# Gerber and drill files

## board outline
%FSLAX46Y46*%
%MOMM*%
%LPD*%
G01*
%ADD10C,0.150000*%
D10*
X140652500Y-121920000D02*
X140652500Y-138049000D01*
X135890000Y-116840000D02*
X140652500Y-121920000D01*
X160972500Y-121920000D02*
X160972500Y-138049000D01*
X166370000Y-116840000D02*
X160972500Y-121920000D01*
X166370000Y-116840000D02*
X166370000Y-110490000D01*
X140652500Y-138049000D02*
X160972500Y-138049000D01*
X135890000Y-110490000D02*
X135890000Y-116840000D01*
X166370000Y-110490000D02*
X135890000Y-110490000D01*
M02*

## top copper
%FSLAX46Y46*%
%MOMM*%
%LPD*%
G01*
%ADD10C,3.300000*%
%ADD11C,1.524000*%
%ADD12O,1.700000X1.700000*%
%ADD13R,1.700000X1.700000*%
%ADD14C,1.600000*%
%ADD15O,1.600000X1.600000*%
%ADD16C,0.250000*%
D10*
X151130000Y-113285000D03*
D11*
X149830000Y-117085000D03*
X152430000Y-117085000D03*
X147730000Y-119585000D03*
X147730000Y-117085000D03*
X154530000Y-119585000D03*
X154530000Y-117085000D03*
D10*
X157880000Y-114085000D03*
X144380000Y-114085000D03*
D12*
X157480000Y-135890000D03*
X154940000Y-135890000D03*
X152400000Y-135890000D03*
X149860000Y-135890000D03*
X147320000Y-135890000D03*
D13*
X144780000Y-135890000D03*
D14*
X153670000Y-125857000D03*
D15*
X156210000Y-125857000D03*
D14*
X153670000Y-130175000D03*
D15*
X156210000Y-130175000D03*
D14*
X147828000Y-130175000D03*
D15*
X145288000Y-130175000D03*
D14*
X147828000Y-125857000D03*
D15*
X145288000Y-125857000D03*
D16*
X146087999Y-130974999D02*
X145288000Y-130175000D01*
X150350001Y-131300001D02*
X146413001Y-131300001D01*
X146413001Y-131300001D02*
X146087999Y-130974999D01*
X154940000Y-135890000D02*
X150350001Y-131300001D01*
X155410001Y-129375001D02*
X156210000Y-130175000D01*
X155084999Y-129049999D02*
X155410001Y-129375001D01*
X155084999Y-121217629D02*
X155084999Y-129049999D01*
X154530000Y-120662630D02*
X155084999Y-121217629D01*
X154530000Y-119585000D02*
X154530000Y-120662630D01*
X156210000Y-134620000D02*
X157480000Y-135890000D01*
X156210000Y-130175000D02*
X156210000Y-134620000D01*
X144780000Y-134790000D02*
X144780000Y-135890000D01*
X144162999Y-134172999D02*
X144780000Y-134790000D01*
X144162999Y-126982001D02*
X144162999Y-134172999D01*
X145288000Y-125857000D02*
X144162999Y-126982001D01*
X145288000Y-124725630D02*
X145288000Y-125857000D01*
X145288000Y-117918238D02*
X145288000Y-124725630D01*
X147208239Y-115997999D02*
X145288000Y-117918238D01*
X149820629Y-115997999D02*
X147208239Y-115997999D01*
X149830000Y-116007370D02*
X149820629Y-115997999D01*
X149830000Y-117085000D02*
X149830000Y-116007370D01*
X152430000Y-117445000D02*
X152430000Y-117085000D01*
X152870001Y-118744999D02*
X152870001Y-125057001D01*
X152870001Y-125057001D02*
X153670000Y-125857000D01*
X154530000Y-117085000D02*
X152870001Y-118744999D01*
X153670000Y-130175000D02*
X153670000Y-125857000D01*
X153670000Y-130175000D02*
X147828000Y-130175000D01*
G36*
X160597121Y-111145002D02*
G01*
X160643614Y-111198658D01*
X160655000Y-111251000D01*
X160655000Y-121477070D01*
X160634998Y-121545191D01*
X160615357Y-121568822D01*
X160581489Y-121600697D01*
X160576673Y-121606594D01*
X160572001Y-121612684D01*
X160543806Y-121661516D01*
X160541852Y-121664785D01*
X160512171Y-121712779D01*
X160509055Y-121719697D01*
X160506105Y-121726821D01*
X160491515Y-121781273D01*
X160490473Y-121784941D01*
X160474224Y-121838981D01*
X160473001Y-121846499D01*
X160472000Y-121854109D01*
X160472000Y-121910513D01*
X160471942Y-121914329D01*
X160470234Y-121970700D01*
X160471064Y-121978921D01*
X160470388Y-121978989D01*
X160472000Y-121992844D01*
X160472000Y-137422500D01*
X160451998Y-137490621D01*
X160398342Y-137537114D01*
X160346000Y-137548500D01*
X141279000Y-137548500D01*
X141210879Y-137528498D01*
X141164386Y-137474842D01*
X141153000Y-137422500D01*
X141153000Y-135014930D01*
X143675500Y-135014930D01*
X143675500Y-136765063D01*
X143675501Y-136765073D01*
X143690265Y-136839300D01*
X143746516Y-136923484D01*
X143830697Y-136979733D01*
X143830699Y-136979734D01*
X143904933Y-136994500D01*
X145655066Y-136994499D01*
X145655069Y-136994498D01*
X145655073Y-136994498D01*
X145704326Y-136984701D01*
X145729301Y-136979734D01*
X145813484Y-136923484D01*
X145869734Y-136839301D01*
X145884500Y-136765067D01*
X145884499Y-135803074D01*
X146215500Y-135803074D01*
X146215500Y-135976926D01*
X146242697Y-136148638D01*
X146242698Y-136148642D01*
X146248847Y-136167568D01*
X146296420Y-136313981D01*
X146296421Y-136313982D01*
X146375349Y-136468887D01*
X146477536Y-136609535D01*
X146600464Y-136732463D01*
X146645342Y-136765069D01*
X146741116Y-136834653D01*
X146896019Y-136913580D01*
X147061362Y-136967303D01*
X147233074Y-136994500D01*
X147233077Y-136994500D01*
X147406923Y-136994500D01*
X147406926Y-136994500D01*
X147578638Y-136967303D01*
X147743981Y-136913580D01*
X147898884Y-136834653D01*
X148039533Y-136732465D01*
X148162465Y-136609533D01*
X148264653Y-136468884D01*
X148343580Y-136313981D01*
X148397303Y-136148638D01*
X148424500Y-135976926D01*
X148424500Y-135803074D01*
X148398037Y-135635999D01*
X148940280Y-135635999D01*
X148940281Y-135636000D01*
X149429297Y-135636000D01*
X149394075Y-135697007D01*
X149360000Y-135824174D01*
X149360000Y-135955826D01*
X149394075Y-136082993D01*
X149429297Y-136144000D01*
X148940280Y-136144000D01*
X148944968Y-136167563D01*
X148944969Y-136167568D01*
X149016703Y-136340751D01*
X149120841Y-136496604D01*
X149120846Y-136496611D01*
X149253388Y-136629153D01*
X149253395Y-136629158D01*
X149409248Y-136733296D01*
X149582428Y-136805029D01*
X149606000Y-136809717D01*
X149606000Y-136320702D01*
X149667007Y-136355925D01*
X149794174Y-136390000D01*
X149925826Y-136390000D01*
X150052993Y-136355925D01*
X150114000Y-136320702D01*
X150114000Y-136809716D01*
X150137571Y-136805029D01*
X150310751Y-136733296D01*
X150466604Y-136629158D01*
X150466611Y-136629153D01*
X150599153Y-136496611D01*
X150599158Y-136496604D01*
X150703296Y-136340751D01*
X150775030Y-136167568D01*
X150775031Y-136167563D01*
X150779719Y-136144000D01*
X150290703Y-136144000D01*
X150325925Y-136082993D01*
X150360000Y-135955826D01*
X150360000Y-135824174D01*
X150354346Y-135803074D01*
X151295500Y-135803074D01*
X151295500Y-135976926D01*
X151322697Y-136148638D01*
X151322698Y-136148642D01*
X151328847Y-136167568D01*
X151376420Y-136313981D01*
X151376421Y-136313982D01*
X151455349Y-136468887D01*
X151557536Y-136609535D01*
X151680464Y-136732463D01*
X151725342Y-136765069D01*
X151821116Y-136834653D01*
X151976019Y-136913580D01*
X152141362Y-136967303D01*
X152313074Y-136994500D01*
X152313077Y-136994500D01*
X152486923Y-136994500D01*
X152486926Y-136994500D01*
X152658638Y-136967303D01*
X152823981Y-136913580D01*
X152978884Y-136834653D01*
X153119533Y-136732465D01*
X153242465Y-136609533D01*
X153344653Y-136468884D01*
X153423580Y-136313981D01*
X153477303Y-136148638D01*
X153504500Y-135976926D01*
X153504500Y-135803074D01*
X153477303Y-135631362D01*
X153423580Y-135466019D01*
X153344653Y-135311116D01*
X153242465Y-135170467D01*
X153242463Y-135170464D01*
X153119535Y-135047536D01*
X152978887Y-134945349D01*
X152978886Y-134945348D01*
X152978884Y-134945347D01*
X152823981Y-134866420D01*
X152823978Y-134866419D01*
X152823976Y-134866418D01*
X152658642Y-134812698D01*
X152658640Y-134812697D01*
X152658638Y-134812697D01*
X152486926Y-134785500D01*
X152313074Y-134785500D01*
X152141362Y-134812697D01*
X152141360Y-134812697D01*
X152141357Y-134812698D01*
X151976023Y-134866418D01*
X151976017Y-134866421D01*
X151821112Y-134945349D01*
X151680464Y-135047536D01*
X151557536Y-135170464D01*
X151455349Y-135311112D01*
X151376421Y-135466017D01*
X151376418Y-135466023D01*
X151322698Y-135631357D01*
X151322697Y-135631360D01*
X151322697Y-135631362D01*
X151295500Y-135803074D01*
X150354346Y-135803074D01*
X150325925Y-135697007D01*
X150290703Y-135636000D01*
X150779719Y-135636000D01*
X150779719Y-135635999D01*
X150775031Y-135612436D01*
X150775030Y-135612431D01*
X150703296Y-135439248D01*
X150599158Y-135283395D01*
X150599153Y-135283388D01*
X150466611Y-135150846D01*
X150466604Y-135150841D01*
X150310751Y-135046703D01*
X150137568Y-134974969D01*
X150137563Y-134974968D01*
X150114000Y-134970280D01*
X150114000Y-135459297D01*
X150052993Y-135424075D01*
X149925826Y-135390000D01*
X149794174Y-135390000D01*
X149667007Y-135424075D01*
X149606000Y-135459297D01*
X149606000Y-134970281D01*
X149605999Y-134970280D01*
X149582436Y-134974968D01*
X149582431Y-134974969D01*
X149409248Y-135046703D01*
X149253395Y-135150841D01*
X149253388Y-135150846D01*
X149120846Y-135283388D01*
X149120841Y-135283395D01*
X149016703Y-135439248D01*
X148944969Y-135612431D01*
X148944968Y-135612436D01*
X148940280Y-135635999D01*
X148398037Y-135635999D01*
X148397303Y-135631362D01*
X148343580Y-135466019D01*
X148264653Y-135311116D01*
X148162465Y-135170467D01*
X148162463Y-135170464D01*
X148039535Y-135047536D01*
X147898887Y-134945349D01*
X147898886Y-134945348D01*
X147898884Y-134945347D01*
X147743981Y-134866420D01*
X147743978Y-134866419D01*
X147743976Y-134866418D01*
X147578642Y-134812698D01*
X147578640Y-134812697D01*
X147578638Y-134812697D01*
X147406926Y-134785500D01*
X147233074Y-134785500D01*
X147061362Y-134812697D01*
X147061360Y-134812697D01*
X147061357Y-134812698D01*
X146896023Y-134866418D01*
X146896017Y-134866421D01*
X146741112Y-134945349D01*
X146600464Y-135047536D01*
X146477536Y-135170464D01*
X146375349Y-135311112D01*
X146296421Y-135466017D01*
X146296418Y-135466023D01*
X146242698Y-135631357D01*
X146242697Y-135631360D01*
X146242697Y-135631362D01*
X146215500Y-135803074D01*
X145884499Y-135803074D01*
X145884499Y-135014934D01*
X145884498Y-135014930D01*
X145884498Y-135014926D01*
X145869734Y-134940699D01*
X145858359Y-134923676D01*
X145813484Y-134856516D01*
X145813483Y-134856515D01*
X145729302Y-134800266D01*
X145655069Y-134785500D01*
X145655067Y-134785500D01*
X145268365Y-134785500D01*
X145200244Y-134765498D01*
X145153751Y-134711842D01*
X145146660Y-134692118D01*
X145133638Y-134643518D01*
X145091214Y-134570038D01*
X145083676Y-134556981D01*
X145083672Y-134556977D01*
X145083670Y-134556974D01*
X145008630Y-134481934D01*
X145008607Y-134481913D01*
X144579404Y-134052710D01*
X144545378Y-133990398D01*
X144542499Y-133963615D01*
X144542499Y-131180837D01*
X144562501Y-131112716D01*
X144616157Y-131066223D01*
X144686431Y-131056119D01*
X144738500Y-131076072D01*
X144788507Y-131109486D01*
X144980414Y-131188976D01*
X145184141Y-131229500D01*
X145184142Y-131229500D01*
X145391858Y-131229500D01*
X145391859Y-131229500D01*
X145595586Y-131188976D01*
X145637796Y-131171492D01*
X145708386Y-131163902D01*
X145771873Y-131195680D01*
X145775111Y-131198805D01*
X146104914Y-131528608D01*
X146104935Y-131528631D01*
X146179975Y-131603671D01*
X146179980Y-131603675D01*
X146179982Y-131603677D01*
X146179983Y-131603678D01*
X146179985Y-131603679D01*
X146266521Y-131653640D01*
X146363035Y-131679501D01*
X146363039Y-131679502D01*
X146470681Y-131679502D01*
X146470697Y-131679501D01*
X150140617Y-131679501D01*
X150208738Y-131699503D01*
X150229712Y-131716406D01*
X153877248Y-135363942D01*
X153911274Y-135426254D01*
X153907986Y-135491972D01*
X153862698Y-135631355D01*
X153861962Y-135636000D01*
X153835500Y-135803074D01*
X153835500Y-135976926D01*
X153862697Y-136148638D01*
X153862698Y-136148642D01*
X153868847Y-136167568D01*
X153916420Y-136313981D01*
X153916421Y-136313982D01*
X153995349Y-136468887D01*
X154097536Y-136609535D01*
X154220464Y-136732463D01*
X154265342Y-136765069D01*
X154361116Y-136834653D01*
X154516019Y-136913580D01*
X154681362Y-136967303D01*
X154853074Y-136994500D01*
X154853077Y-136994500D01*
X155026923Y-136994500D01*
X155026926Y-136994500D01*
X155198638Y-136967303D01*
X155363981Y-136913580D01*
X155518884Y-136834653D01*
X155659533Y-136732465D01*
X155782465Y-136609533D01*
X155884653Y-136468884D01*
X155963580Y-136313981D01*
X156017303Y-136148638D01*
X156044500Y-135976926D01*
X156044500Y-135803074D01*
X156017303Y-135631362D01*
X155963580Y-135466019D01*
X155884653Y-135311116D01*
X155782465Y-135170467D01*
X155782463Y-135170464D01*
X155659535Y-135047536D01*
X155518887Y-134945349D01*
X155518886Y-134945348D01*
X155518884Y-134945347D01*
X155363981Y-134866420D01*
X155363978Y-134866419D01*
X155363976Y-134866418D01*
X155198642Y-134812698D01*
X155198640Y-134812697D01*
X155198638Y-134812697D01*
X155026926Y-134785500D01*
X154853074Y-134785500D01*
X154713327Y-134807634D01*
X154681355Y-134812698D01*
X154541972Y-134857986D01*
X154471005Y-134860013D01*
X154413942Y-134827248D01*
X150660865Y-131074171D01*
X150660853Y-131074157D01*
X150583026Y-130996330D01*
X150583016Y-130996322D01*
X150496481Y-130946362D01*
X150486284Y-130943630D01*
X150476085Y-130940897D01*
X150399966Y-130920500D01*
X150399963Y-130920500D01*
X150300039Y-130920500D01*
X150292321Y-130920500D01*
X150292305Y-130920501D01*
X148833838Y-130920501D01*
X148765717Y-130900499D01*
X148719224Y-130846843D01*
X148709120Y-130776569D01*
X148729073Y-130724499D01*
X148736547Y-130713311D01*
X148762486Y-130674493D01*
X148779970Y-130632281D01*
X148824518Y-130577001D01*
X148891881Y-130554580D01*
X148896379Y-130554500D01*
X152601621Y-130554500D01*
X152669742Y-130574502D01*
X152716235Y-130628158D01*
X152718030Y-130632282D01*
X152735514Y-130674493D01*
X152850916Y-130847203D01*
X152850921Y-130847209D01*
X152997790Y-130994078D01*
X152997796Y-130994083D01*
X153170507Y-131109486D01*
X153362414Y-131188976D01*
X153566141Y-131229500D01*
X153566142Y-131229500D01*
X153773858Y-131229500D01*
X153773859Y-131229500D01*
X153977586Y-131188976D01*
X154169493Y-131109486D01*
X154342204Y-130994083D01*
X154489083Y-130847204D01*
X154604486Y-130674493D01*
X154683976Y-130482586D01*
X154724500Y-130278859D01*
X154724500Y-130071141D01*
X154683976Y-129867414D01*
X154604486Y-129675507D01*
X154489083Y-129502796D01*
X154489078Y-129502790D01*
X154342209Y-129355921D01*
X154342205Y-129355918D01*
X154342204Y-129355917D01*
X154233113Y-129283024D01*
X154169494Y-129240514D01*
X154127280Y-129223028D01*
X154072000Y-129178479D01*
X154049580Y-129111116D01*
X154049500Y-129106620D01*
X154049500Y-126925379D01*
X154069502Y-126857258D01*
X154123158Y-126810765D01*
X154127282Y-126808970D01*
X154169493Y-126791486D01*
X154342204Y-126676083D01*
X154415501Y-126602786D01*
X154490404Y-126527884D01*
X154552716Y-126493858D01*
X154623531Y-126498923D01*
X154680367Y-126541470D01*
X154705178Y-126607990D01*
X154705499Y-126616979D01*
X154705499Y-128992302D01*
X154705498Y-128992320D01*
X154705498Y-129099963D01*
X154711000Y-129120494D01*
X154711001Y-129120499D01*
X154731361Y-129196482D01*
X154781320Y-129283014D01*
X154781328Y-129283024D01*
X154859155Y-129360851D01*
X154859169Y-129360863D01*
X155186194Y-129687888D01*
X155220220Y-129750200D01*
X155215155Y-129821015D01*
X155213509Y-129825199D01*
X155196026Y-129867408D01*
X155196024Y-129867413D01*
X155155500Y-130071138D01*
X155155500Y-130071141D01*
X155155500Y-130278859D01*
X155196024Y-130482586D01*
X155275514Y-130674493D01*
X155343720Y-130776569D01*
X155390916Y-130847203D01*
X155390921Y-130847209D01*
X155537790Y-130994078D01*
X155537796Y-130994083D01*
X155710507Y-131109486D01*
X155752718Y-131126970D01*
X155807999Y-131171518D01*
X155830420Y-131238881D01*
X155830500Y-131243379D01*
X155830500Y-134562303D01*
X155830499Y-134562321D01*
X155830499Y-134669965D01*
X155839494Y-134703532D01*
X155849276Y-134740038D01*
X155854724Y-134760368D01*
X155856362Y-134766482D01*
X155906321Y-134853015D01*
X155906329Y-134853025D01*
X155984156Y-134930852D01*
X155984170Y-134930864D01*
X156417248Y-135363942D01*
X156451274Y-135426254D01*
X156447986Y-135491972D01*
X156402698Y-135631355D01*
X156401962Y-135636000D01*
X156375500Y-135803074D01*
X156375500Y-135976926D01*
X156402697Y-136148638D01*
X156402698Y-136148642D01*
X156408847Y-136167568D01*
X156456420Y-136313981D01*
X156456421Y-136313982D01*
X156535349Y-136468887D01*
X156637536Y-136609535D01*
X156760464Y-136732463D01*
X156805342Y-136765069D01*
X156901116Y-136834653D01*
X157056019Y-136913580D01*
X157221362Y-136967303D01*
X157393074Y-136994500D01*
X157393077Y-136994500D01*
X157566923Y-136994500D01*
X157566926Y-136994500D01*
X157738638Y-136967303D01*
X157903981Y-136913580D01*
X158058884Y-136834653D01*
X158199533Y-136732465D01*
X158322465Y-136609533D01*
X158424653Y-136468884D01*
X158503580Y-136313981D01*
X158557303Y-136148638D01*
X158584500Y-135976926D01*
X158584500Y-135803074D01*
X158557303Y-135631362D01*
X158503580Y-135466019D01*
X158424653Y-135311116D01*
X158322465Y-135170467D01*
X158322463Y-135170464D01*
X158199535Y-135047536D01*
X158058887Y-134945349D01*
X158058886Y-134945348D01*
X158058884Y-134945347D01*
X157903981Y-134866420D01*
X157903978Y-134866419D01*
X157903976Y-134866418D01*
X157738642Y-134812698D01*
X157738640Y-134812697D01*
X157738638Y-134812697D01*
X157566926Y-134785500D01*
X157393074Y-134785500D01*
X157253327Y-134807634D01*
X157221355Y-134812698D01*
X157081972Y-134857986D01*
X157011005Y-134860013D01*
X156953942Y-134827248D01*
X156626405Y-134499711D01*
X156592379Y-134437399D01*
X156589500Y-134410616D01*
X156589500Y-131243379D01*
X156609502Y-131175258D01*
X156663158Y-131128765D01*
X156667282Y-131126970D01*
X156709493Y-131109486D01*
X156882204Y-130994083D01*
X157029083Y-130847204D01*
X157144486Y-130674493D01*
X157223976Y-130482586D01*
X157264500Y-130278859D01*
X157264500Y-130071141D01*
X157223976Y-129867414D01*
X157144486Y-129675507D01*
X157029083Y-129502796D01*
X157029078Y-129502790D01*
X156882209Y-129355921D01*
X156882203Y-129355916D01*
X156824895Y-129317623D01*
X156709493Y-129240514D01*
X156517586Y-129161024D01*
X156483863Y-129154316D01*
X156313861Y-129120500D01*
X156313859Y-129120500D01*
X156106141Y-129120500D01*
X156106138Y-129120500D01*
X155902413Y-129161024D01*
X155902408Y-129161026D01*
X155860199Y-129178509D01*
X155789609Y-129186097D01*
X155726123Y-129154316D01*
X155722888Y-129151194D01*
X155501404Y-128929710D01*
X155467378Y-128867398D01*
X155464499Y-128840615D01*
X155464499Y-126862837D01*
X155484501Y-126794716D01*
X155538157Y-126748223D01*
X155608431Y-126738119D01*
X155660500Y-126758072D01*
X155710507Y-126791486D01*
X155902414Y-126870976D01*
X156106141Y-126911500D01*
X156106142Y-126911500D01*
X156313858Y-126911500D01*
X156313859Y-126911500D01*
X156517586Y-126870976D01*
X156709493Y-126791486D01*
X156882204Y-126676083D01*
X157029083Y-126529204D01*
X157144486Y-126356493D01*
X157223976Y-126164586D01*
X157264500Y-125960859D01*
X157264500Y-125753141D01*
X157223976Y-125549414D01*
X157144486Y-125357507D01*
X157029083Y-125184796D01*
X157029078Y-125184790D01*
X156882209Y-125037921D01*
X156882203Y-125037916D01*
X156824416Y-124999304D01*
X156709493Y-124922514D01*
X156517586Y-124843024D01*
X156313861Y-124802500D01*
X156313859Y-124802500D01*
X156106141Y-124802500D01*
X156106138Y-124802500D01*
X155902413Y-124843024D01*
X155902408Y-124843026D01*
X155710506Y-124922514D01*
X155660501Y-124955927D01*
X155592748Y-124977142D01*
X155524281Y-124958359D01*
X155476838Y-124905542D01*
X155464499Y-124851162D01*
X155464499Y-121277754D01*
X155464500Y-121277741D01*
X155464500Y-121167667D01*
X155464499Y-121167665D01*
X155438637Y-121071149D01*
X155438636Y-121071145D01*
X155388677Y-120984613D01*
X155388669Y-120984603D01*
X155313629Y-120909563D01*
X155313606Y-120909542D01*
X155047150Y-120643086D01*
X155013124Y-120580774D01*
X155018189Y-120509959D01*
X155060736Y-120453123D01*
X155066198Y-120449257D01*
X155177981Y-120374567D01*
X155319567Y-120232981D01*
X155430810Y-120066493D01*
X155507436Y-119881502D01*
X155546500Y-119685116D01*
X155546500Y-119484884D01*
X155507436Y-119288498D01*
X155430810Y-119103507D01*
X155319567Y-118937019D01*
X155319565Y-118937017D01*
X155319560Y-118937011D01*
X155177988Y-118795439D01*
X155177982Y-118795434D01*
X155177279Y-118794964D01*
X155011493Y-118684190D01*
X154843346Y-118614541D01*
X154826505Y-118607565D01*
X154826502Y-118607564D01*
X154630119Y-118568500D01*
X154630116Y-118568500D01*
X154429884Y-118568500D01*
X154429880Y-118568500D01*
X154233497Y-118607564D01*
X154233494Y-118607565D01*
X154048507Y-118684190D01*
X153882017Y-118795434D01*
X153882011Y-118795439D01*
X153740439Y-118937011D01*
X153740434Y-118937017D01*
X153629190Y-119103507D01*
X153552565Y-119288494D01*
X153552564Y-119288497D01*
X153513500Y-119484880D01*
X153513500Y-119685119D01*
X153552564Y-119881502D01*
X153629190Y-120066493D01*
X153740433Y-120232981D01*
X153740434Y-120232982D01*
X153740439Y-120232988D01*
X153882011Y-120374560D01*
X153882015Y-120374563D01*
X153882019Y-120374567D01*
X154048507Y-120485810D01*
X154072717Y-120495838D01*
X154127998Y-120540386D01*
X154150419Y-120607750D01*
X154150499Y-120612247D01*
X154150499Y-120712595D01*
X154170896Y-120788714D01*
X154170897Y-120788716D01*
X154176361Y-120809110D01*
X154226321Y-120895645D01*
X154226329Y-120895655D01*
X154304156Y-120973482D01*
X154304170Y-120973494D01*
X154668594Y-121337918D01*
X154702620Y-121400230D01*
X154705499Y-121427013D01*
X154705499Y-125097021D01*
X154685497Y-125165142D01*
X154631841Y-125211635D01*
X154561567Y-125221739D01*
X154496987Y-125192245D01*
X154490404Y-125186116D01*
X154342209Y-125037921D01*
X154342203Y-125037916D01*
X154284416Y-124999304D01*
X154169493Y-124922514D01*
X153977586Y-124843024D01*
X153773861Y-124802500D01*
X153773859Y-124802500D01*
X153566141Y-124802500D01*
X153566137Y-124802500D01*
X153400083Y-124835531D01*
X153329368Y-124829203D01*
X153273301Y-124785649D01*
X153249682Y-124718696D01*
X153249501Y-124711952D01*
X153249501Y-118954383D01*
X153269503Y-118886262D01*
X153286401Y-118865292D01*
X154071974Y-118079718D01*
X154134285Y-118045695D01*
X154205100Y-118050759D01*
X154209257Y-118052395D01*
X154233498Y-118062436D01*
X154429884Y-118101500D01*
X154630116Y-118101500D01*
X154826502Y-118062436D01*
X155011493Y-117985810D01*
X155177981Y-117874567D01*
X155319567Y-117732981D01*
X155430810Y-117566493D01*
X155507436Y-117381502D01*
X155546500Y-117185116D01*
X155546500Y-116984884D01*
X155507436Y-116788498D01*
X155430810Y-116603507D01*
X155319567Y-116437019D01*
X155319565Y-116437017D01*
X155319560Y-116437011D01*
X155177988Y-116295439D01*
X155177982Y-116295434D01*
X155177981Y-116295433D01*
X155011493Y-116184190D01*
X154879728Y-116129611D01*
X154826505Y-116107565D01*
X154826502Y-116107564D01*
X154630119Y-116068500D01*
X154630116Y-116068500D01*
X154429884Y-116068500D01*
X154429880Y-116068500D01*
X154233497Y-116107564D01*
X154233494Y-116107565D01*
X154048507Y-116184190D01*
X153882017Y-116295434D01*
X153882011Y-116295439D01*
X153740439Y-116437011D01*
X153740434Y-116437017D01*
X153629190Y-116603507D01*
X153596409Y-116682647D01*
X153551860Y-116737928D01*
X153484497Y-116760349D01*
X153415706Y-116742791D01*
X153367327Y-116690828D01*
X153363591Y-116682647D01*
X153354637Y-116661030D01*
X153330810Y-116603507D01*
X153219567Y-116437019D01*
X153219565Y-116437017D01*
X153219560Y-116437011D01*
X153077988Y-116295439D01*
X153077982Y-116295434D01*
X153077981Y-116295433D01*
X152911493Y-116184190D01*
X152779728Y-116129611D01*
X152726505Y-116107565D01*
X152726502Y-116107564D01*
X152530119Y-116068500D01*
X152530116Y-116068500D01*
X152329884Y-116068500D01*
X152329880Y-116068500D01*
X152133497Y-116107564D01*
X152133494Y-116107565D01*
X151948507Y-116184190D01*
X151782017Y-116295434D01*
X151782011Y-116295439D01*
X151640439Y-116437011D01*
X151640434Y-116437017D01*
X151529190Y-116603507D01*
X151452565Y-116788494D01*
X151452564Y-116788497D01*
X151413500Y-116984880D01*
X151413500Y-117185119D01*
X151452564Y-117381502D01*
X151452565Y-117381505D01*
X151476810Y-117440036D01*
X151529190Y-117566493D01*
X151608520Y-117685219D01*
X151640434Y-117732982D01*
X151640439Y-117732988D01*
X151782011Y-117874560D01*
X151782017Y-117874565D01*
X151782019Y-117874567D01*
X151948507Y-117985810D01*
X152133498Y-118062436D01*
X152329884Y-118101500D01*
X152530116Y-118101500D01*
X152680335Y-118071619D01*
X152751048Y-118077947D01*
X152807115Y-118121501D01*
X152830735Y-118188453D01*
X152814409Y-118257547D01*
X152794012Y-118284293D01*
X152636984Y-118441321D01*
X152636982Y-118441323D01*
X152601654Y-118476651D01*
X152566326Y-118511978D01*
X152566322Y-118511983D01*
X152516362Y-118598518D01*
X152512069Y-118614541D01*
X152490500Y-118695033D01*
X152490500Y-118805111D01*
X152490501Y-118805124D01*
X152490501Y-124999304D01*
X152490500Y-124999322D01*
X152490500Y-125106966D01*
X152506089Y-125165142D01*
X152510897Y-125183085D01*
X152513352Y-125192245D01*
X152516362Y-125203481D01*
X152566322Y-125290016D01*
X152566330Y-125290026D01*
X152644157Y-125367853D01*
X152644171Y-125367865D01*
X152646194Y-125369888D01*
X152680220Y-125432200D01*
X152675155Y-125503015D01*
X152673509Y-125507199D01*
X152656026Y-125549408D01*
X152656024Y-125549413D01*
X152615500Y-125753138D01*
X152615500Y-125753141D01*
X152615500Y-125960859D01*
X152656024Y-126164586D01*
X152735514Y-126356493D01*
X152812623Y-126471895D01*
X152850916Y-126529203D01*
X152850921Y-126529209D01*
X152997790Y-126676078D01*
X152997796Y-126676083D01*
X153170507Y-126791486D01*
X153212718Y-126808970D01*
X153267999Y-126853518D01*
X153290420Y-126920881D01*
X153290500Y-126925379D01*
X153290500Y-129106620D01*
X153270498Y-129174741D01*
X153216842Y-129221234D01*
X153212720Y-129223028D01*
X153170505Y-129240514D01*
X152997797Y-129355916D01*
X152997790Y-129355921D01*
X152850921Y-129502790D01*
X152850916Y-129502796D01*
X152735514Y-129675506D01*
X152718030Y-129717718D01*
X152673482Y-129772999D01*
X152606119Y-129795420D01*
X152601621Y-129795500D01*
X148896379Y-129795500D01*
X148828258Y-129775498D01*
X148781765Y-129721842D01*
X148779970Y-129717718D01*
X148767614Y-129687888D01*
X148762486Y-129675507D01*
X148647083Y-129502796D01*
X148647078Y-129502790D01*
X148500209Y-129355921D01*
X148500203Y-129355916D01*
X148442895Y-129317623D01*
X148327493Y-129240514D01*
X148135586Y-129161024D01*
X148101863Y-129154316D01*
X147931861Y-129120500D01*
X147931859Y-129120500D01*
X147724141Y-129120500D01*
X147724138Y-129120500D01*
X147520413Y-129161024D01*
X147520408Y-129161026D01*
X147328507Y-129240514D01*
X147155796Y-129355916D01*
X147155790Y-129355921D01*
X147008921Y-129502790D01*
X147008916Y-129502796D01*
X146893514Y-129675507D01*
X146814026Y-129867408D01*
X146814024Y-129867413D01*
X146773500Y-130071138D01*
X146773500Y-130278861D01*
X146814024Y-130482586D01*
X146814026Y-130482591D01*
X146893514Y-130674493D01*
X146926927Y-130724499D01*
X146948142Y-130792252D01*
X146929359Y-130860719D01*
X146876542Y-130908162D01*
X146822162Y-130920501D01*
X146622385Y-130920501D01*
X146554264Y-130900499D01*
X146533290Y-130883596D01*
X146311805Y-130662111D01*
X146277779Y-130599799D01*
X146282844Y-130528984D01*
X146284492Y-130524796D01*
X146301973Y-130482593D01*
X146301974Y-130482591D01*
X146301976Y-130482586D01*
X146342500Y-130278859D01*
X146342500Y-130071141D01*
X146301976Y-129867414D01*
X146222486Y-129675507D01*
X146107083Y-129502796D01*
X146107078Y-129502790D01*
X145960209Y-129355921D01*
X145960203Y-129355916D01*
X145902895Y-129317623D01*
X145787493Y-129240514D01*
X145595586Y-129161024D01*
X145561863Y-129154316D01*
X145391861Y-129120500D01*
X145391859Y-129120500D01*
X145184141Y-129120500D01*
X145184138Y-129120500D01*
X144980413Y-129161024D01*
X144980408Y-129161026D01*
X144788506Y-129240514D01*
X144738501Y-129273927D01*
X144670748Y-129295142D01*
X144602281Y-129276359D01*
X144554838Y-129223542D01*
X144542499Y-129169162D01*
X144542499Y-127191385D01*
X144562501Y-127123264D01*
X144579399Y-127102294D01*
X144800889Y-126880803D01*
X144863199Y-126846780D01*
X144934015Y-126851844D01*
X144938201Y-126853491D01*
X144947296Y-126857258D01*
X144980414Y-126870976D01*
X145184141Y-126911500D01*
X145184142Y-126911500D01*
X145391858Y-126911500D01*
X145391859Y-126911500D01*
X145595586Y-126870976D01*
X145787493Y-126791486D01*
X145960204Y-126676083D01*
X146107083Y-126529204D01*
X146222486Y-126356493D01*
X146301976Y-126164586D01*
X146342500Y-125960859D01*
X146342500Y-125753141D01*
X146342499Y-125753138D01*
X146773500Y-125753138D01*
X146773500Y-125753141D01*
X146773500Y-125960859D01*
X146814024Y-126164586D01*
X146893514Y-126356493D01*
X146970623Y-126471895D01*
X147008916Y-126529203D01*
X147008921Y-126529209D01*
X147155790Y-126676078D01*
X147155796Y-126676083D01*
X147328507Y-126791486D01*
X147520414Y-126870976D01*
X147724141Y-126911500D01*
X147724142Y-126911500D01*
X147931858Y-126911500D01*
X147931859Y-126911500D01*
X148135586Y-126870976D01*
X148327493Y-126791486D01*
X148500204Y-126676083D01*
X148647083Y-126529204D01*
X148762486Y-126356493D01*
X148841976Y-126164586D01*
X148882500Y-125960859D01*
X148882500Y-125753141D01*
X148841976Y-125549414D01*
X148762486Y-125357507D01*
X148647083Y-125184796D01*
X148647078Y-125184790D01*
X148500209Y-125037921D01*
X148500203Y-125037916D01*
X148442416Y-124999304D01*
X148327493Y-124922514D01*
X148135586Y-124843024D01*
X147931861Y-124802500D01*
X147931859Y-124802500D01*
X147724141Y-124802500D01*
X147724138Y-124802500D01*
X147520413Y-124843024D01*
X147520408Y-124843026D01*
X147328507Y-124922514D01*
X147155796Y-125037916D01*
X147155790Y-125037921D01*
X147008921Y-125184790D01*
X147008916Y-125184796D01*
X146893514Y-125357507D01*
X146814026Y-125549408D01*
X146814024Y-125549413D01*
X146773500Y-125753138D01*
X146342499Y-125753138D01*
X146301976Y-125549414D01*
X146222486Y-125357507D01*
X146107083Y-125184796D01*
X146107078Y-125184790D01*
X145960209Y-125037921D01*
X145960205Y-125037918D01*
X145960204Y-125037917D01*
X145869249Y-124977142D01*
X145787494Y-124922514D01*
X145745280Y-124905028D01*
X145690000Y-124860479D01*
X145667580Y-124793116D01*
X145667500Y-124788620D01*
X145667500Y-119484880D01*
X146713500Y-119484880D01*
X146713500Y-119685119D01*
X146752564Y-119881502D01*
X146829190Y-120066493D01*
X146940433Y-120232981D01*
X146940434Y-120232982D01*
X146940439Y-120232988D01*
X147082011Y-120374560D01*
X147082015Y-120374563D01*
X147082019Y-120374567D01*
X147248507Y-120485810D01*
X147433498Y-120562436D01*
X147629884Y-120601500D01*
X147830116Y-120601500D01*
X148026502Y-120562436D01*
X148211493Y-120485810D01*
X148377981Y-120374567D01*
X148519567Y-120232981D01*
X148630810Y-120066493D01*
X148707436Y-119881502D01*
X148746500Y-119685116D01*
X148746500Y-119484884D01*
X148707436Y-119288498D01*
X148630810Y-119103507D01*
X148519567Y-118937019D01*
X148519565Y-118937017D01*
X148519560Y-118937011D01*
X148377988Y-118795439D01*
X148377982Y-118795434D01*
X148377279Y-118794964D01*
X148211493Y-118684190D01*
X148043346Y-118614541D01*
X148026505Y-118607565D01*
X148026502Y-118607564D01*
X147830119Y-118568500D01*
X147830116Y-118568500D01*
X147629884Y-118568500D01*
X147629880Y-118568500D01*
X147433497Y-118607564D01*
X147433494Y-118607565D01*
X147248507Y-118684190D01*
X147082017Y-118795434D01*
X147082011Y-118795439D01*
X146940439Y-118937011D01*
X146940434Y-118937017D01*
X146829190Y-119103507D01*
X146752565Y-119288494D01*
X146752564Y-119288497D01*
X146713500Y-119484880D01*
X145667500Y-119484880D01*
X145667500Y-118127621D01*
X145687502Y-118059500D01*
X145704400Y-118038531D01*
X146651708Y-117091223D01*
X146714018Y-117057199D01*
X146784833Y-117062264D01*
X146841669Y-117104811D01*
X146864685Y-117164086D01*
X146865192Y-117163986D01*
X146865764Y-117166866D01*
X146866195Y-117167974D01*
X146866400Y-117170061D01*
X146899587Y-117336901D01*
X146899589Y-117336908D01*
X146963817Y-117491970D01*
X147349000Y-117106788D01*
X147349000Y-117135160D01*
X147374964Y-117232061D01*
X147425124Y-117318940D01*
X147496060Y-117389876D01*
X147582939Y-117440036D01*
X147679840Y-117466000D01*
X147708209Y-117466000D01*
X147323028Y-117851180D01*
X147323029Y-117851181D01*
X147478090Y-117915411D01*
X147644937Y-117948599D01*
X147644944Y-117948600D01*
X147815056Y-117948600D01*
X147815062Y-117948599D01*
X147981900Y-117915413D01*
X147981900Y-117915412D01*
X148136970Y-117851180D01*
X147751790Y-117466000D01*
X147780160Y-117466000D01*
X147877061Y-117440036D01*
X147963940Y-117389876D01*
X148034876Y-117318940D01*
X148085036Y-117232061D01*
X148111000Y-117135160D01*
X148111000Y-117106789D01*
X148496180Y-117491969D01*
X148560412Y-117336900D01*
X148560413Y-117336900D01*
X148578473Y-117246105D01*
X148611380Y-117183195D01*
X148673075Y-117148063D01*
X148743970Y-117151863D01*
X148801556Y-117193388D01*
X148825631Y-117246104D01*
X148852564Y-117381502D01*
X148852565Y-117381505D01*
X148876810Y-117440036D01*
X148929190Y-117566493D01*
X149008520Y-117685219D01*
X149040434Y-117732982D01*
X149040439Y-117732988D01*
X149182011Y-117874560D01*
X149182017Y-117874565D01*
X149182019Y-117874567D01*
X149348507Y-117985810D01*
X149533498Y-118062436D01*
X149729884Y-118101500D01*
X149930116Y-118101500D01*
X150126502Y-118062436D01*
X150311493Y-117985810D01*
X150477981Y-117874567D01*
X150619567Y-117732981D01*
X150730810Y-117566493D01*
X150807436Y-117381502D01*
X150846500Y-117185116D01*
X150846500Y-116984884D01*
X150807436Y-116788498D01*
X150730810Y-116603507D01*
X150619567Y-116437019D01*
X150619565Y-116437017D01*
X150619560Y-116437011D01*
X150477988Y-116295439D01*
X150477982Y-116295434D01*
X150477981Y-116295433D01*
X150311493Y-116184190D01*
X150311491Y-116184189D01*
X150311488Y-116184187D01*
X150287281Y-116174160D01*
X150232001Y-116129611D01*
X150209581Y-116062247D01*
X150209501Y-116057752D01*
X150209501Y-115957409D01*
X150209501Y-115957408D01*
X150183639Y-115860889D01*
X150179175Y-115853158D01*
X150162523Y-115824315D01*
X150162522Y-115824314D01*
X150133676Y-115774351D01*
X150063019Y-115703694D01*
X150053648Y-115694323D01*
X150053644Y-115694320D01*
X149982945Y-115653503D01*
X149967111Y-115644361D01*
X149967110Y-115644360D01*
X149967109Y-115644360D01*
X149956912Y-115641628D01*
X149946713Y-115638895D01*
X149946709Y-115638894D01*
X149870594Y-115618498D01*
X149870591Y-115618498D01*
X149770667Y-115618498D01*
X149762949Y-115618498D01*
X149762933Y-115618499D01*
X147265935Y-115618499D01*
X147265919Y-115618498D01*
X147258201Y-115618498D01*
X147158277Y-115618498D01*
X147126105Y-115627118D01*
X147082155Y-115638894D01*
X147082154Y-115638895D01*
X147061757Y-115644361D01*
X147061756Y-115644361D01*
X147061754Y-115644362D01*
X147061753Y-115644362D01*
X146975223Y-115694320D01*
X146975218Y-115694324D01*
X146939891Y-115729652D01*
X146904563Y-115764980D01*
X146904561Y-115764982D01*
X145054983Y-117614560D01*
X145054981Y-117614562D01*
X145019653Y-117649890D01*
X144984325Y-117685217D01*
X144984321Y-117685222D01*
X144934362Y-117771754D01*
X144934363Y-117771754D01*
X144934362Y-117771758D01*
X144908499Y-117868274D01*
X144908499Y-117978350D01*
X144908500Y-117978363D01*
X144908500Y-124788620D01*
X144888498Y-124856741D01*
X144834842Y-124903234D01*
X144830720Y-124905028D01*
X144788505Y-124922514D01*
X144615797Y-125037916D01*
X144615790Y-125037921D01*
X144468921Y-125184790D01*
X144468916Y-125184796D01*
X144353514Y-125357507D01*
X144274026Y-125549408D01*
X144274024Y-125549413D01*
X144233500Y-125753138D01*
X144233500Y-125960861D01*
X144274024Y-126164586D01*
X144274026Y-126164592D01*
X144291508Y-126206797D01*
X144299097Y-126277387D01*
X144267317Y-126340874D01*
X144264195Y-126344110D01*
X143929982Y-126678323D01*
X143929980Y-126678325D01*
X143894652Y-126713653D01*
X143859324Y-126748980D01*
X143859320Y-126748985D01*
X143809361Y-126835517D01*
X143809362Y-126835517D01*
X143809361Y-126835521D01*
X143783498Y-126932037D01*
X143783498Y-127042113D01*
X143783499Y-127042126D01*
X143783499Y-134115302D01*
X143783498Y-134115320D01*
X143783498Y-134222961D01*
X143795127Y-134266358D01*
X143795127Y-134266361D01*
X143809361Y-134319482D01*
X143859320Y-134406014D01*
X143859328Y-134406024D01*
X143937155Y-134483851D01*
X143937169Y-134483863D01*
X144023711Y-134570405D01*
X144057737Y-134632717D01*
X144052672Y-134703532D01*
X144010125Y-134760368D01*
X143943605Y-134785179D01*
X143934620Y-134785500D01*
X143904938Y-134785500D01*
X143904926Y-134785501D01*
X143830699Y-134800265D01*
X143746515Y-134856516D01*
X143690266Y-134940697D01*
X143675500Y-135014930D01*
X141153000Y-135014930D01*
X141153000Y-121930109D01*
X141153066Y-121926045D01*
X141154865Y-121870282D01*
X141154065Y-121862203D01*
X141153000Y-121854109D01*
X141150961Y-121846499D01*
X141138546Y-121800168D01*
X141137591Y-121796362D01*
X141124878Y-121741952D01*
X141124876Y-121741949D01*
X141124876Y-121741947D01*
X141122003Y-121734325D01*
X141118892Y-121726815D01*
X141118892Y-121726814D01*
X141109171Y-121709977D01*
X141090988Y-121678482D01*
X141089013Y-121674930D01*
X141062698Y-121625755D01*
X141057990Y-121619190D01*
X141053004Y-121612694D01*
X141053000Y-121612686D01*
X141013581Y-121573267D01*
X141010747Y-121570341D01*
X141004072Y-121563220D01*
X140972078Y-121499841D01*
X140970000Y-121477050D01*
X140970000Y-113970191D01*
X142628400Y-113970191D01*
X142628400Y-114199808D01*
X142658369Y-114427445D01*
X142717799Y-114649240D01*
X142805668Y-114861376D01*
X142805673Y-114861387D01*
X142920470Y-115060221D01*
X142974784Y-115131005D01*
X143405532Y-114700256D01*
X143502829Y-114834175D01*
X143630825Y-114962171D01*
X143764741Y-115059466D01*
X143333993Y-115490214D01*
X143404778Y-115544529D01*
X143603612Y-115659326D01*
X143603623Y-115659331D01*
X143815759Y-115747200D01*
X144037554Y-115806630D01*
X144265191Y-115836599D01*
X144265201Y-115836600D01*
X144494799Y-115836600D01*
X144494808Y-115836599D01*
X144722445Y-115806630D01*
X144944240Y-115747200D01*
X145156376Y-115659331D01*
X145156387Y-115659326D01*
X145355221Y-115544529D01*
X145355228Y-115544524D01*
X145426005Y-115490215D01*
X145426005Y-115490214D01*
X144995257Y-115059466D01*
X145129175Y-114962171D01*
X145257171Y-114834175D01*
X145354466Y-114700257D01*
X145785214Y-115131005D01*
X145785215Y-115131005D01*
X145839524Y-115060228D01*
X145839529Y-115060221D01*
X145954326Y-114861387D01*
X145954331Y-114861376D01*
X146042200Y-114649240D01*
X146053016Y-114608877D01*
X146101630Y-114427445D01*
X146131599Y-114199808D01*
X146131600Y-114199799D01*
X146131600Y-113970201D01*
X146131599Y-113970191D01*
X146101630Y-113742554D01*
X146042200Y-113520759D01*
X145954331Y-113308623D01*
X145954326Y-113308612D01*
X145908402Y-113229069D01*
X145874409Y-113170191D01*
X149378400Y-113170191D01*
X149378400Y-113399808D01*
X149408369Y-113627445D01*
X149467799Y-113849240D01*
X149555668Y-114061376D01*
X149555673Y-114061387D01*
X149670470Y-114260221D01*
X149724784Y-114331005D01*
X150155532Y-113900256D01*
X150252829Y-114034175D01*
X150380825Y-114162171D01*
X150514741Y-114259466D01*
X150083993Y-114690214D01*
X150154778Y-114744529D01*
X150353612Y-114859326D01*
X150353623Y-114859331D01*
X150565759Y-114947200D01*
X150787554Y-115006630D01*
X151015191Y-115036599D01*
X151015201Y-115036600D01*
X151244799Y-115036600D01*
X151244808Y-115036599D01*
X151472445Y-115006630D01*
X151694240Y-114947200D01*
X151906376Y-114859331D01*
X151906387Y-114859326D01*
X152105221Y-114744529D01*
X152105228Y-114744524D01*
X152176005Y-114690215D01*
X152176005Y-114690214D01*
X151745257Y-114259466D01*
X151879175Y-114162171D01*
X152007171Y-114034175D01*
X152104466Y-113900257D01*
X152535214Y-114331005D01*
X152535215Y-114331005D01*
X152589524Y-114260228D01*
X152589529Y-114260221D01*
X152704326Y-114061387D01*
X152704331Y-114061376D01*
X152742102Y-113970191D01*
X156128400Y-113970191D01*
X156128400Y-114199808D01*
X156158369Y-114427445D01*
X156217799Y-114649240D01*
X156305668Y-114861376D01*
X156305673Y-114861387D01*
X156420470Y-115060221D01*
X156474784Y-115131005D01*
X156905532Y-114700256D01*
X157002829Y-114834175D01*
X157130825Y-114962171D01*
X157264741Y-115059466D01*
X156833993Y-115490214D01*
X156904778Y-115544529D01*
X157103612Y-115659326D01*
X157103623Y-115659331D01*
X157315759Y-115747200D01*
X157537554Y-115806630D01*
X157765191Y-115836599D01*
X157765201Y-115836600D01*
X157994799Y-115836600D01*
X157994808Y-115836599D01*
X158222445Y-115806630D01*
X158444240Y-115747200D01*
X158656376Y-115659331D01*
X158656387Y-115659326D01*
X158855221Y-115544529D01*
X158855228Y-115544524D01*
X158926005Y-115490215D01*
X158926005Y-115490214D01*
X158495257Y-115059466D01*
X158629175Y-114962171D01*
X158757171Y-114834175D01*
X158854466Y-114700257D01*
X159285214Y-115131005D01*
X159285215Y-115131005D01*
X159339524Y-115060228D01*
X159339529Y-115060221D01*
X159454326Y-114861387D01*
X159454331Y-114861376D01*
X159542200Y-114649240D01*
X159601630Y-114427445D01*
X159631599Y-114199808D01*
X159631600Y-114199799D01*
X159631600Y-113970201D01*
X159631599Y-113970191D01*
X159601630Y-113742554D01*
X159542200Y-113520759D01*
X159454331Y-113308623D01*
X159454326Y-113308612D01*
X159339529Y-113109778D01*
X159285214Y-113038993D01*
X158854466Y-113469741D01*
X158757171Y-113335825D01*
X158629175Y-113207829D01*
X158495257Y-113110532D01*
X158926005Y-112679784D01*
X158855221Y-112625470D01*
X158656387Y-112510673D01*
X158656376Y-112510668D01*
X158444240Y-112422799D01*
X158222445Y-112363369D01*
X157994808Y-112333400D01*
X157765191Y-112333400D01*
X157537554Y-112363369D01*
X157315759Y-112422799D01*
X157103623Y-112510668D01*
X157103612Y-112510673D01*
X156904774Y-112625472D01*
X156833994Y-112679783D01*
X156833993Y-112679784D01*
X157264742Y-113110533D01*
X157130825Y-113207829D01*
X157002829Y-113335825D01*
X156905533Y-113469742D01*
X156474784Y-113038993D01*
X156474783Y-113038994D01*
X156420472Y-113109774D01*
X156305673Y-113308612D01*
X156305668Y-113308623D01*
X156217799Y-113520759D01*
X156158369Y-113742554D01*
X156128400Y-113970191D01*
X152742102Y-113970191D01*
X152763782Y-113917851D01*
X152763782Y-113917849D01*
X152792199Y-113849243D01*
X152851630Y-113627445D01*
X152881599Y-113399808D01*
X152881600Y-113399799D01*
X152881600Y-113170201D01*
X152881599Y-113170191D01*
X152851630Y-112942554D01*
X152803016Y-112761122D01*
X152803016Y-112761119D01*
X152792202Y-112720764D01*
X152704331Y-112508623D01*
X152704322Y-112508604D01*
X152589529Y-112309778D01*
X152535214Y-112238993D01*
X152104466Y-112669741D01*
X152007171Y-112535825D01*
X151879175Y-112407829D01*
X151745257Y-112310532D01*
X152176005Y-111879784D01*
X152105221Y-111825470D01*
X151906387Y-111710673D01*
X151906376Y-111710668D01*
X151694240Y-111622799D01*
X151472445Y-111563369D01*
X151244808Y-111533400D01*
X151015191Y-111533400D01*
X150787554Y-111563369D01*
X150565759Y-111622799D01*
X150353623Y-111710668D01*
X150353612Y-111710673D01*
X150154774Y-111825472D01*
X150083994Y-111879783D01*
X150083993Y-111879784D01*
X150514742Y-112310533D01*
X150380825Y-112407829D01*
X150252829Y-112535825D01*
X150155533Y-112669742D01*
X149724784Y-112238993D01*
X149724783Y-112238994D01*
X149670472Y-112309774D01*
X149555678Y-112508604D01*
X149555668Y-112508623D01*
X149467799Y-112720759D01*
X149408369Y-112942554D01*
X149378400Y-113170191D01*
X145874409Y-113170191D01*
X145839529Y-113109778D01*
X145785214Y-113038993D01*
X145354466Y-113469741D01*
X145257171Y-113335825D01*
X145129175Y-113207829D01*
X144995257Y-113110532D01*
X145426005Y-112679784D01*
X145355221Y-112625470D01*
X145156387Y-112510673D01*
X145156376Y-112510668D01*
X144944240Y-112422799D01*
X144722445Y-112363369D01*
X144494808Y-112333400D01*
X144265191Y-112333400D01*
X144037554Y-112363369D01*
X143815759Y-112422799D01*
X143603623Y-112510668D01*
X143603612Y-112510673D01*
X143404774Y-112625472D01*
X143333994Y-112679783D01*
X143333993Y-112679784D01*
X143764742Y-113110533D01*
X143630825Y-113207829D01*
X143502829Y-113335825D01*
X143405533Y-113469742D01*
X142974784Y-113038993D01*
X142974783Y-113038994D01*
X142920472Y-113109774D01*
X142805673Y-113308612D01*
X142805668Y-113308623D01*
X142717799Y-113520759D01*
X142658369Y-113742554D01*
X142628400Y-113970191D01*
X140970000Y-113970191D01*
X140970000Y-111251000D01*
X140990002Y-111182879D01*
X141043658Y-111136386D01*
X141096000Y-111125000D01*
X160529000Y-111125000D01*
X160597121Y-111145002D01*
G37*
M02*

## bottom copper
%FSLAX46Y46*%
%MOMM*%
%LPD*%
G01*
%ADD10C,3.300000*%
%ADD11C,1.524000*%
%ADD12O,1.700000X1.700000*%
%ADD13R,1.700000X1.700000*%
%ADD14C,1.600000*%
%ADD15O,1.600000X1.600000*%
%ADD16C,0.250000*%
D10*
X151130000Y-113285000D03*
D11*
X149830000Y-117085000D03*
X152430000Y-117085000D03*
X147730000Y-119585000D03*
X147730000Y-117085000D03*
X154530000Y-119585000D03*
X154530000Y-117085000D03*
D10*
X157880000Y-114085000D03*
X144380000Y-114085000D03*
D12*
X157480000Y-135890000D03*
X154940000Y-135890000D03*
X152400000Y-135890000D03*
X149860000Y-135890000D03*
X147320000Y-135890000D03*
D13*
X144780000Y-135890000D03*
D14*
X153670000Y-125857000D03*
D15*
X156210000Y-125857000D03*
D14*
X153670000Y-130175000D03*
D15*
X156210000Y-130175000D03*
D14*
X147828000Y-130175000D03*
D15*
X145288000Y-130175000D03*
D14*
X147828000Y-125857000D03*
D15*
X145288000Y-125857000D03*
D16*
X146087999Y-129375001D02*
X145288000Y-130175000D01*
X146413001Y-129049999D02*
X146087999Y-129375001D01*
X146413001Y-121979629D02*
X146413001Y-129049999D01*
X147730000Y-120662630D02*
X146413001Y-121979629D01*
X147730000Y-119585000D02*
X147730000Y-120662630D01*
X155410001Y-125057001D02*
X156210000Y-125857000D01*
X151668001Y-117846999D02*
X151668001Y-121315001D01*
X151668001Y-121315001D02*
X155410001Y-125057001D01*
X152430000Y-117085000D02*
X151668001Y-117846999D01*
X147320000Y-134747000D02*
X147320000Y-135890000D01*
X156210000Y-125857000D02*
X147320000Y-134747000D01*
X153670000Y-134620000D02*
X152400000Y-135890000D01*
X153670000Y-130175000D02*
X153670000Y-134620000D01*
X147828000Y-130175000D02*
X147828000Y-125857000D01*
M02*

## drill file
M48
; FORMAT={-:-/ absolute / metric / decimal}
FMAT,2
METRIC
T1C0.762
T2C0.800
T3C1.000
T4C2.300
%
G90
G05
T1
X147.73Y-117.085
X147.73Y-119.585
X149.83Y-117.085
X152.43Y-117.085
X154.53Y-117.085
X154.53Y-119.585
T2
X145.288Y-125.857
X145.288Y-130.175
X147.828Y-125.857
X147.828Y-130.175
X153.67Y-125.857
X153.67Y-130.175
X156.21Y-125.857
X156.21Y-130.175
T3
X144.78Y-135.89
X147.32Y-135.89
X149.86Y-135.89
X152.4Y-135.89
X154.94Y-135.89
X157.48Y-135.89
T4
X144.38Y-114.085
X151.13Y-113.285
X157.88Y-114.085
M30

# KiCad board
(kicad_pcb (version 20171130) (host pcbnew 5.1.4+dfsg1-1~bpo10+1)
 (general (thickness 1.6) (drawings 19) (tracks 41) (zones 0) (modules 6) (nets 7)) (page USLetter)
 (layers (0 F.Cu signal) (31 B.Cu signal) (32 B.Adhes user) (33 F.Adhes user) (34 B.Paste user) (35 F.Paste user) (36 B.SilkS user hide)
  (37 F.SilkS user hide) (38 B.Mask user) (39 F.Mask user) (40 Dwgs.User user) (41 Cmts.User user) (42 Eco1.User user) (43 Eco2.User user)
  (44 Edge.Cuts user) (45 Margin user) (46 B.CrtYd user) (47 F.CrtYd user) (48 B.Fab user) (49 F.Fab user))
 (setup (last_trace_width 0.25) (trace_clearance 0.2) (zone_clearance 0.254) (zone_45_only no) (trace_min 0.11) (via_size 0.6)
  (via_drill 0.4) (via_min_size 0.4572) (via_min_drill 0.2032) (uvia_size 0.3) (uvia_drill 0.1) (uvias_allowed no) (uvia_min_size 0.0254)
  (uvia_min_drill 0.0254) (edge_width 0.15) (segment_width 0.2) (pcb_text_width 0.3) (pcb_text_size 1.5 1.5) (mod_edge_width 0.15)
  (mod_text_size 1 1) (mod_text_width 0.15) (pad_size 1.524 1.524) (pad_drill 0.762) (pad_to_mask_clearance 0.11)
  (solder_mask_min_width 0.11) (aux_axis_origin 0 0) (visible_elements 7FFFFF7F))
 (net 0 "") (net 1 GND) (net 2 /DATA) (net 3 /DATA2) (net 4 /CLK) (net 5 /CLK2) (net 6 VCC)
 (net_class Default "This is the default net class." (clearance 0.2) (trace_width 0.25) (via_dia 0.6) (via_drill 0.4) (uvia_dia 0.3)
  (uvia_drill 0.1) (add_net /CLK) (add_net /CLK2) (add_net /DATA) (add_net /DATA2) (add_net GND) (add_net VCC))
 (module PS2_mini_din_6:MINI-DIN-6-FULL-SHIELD (layer F.Cu) (at 151.13 108.585)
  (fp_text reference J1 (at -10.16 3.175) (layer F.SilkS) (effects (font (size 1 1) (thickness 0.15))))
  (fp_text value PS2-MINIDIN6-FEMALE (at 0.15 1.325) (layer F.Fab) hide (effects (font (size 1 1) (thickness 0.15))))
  (pad 7 thru_hole circle (at 0 4.7) (size 3.3 3.3) (drill 2.3) (layers *.Cu *.Mask) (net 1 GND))
  (pad 1 thru_hole circle (at -1.3 8.5) (size 1.524 1.524) (drill 0.762) (layers *.Cu *.Mask) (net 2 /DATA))
  (pad 2 thru_hole circle (at 1.3 8.5) (size 1.524 1.524) (drill 0.762) (layers *.Cu *.Mask) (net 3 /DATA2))
  (pad 5 thru_hole circle (at -3.4 11) (size 1.524 1.524) (drill 0.762) (layers *.Cu *.Mask) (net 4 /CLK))
  (pad 3 thru_hole circle (at -3.4 8.5) (size 1.524 1.524) (drill 0.762) (layers *.Cu *.Mask) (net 1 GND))
  (pad 6 thru_hole circle (at 3.4 11) (size 1.524 1.524) (drill 0.762) (layers *.Cu *.Mask) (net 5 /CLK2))
  (pad 4 thru_hole circle (at 3.4 8.5) (size 1.524 1.524) (drill 0.762) (layers *.Cu *.Mask) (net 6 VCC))
  (pad 7 thru_hole circle (at 6.75 5.5) (size 3.3 3.3) (drill 2.3) (layers *.Cu *.Mask) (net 1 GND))
  (pad 7 thru_hole circle (at -6.75 5.5) (size 3.3 3.3) (drill 2.3) (layers *.Cu *.Mask) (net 1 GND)))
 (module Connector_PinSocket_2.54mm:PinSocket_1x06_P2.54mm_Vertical (layer F.Cu) (at 144.78 135.89 90)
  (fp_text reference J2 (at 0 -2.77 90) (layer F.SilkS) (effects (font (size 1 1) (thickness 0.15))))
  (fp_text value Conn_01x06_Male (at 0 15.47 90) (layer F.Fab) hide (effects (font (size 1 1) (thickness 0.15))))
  (pad 6 thru_hole oval (at 0 12.7 90) (size 1.7 1.7) (drill 1) (layers *.Cu *.Mask) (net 5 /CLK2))
  (pad 5 thru_hole oval (at 0 10.16 90) (size 1.7 1.7) (drill 1) (layers *.Cu *.Mask) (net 4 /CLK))
  (pad 4 thru_hole oval (at 0 7.62 90) (size 1.7 1.7) (drill 1) (layers *.Cu *.Mask) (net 6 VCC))
  (pad 3 thru_hole oval (at 0 5.08 90) (size 1.7 1.7) (drill 1) (layers *.Cu *.Mask) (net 1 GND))
  (pad 2 thru_hole oval (at 0 2.54 90) (size 1.7 1.7) (drill 1) (layers *.Cu *.Mask) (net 3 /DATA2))
  (pad 1 thru_hole rect (at 0 0 90) (size 1.7 1.7) (drill 1) (layers *.Cu *.Mask) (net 2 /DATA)))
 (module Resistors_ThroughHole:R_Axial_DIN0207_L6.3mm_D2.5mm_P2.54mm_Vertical (layer F.Cu) (at 153.67 125.857)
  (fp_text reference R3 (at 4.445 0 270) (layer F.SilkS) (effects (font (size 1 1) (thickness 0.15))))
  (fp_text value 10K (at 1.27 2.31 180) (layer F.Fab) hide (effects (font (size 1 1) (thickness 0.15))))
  (pad 1 thru_hole circle (at 0 0) (size 1.6 1.6) (drill 0.8) (layers *.Cu *.Mask) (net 6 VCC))
  (pad 2 thru_hole oval (at 2.54 0) (size 1.6 1.6) (drill 0.8) (layers *.Cu *.Mask) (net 3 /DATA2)))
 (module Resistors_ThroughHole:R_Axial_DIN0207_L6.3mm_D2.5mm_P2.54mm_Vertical (layer F.Cu) (at 153.67 130.175)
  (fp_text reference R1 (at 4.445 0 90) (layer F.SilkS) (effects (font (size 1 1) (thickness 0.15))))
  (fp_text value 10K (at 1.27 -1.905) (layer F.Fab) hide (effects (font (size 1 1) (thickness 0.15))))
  (pad 1 thru_hole circle (at 0 0) (size 1.6 1.6) (drill 0.8) (layers *.Cu *.Mask) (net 6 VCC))
  (pad 2 thru_hole oval (at 2.54 0) (size 1.6 1.6) (drill 0.8) (layers *.Cu *.Mask) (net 5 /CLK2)))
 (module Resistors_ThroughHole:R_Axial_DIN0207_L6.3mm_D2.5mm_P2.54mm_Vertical (layer F.Cu) (at 147.828 130.175 180)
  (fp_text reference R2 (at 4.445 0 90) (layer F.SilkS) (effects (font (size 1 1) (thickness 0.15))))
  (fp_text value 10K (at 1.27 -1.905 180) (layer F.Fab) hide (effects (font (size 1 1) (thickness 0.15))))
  (pad 1 thru_hole circle (at 0 0 180) (size 1.6 1.6) (drill 0.8) (layers *.Cu *.Mask) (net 6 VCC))
  (pad 2 thru_hole oval (at 2.54 0 180) (size 1.6 1.6) (drill 0.8) (layers *.Cu *.Mask) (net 4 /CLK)))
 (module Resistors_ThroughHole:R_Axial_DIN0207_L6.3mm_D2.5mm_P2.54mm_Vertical (layer F.Cu) (at 147.828 125.857 180)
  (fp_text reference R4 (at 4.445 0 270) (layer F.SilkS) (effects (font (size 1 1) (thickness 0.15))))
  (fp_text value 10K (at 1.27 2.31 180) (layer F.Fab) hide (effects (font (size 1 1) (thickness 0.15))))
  (pad 1 thru_hole circle (at 0 0 180) (size 1.6 1.6) (drill 0.8) (layers *.Cu *.Mask) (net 6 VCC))
  (pad 2 thru_hole oval (at 2.54 0 180) (size 1.6 1.6) (drill 0.8) (layers *.Cu *.Mask) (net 2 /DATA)))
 (gr_line (start 140.6525 121.92) (end 140.6525 138.049) (layer Edge.Cuts) (width 0.15))
 (gr_line (start 135.89 116.84) (end 140.6525 121.92) (layer Edge.Cuts) (width 0.15))
 (gr_line (start 160.9725 121.92) (end 160.9725 138.049) (layer Edge.Cuts) (width 0.15))
 (gr_line (start 166.37 116.84) (end 160.9725 121.92) (layer Edge.Cuts) (width 0.15))
 (gr_line (start 166.37 116.84) (end 166.37 110.49) (layer Edge.Cuts) (width 0.15))
 (gr_line (start 140.6525 138.049) (end 160.9725 138.049) (layer Edge.Cuts) (width 0.15))
 (gr_line (start 135.89 110.49) (end 135.89 116.84) (layer Edge.Cuts) (width 0.15))
 (gr_line (start 166.37 110.49) (end 135.89 110.49) (layer Edge.Cuts) (width 0.15))
 (segment (start 146.087999 129.375001) (end 145.288 130.175) (width 0.25) (layer B.Cu) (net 4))
 (segment (start 146.413001 129.049999) (end 146.087999 129.375001) (width 0.25) (layer B.Cu) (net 4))
 (segment (start 146.413001 121.979629) (end 146.413001 129.049999) (width 0.25) (layer B.Cu) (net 4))
 (segment (start 147.73 120.66263) (end 146.413001 121.979629) (width 0.25) (layer B.Cu) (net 4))
 (segment (start 147.73 119.585) (end 147.73 120.66263) (width 0.25) (layer B.Cu) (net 4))
 (segment (start 146.087999 130.974999) (end 145.288 130.175) (width 0.25) (layer F.Cu) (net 4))
 (segment (start 150.350001 131.300001) (end 146.413001 131.300001) (width 0.25) (layer F.Cu) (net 4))
 (segment (start 146.413001 131.300001) (end 146.087999 130.974999) (width 0.25) (layer F.Cu) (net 4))
 (segment (start 154.94 135.89) (end 150.350001 131.300001) (width 0.25) (layer F.Cu) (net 4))
 (segment (start 155.410001 129.375001) (end 156.21 130.175) (width 0.25) (layer F.Cu) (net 5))
 (segment (start 155.084999 129.049999) (end 155.410001 129.375001) (width 0.25) (layer F.Cu) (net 5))
 (segment (start 155.084999 121.217629) (end 155.084999 129.049999) (width 0.25) (layer F.Cu) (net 5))
 (segment (start 154.53 120.66263) (end 155.084999 121.217629) (width 0.25) (layer F.Cu) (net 5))
 (segment (start 154.53 119.585) (end 154.53 120.66263) (width 0.25) (layer F.Cu) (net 5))
 (segment (start 156.21 134.62) (end 157.48 135.89) (width 0.25) (layer F.Cu) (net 5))
 (segment (start 156.21 130.175) (end 156.21 134.62) (width 0.25) (layer F.Cu) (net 5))
 (segment (start 144.78 134.79) (end 144.78 135.89) (width 0.25) (layer F.Cu) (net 2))
 (segment (start 144.162999 134.172999) (end 144.78 134.79) (width 0.25) (layer F.Cu) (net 2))
 (segment (start 144.162999 126.982001) (end 144.162999 134.172999) (width 0.25) (layer F.Cu) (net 2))
 (segment (start 145.288 125.857) (end 144.162999 126.982001) (width 0.25) (layer F.Cu) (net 2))
 (segment (start 145.288 124.72563) (end 145.288 125.857) (width 0.25) (layer F.Cu) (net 2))
 (segment (start 145.288 117.918238) (end 145.288 124.72563) (width 0.25) (layer F.Cu) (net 2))
 (segment (start 147.208239 115.997999) (end 145.288 117.918238) (width 0.25) (layer F.Cu) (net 2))
 (segment (start 149.820629 115.997999) (end 147.208239 115.997999) (width 0.25) (layer F.Cu) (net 2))
 (segment (start 149.83 116.00737) (end 149.820629 115.997999) (width 0.25) (layer F.Cu) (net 2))
 (segment (start 149.83 117.085) (end 149.83 116.00737) (width 0.25) (layer F.Cu) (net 2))
 (segment (start 152.43 117.445) (end 152.43 117.085) (width 0.25) (layer F.Cu) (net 3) (status 30))
 (segment (start 155.410001 125.057001) (end 156.21 125.857) (width 0.25) (layer B.Cu) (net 3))
 (segment (start 151.668001 117.846999) (end 151.668001 121.315001) (width 0.25) (layer B.Cu) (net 3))
 (segment (start 151.668001 121.315001) (end 155.410001 125.057001) (width 0.25) (layer B.Cu) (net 3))
 (segment (start 152.43 117.085) (end 151.668001 117.846999) (width 0.25) (layer B.Cu) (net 3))
 (segment (start 147.32 134.747) (end 147.32 135.89) (width 0.25) (layer B.Cu) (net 3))
 (segment (start 156.21 125.857) (end 147.32 134.747) (width 0.25) (layer B.Cu) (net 3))
 (segment (start 152.870001 118.744999) (end 152.870001 125.057001) (width 0.25) (layer F.Cu) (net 6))
 (segment (start 152.870001 125.057001) (end 153.67 125.857) (width 0.25) (layer F.Cu) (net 6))
 (segment (start 154.53 117.085) (end 152.870001 118.744999) (width 0.25) (layer F.Cu) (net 6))
 (segment (start 153.67 130.175) (end 153.67 125.857) (width 0.25) (layer F.Cu) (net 6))
 (segment (start 153.67 130.175) (end 147.828 130.175) (width 0.25) (layer F.Cu) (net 6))
 (segment (start 153.67 134.62) (end 152.4 135.89) (width 0.25) (layer B.Cu) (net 6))
 (segment (start 153.67 130.175) (end 153.67 134.62) (width 0.25) (layer B.Cu) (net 6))
 (segment (start 147.828 130.175) (end 147.828 125.857) (width 0.25) (layer B.Cu) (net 6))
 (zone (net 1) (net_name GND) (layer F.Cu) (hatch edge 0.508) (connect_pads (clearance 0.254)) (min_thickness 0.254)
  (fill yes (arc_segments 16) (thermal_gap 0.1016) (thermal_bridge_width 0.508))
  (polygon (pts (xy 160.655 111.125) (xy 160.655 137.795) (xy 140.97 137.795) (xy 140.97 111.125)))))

